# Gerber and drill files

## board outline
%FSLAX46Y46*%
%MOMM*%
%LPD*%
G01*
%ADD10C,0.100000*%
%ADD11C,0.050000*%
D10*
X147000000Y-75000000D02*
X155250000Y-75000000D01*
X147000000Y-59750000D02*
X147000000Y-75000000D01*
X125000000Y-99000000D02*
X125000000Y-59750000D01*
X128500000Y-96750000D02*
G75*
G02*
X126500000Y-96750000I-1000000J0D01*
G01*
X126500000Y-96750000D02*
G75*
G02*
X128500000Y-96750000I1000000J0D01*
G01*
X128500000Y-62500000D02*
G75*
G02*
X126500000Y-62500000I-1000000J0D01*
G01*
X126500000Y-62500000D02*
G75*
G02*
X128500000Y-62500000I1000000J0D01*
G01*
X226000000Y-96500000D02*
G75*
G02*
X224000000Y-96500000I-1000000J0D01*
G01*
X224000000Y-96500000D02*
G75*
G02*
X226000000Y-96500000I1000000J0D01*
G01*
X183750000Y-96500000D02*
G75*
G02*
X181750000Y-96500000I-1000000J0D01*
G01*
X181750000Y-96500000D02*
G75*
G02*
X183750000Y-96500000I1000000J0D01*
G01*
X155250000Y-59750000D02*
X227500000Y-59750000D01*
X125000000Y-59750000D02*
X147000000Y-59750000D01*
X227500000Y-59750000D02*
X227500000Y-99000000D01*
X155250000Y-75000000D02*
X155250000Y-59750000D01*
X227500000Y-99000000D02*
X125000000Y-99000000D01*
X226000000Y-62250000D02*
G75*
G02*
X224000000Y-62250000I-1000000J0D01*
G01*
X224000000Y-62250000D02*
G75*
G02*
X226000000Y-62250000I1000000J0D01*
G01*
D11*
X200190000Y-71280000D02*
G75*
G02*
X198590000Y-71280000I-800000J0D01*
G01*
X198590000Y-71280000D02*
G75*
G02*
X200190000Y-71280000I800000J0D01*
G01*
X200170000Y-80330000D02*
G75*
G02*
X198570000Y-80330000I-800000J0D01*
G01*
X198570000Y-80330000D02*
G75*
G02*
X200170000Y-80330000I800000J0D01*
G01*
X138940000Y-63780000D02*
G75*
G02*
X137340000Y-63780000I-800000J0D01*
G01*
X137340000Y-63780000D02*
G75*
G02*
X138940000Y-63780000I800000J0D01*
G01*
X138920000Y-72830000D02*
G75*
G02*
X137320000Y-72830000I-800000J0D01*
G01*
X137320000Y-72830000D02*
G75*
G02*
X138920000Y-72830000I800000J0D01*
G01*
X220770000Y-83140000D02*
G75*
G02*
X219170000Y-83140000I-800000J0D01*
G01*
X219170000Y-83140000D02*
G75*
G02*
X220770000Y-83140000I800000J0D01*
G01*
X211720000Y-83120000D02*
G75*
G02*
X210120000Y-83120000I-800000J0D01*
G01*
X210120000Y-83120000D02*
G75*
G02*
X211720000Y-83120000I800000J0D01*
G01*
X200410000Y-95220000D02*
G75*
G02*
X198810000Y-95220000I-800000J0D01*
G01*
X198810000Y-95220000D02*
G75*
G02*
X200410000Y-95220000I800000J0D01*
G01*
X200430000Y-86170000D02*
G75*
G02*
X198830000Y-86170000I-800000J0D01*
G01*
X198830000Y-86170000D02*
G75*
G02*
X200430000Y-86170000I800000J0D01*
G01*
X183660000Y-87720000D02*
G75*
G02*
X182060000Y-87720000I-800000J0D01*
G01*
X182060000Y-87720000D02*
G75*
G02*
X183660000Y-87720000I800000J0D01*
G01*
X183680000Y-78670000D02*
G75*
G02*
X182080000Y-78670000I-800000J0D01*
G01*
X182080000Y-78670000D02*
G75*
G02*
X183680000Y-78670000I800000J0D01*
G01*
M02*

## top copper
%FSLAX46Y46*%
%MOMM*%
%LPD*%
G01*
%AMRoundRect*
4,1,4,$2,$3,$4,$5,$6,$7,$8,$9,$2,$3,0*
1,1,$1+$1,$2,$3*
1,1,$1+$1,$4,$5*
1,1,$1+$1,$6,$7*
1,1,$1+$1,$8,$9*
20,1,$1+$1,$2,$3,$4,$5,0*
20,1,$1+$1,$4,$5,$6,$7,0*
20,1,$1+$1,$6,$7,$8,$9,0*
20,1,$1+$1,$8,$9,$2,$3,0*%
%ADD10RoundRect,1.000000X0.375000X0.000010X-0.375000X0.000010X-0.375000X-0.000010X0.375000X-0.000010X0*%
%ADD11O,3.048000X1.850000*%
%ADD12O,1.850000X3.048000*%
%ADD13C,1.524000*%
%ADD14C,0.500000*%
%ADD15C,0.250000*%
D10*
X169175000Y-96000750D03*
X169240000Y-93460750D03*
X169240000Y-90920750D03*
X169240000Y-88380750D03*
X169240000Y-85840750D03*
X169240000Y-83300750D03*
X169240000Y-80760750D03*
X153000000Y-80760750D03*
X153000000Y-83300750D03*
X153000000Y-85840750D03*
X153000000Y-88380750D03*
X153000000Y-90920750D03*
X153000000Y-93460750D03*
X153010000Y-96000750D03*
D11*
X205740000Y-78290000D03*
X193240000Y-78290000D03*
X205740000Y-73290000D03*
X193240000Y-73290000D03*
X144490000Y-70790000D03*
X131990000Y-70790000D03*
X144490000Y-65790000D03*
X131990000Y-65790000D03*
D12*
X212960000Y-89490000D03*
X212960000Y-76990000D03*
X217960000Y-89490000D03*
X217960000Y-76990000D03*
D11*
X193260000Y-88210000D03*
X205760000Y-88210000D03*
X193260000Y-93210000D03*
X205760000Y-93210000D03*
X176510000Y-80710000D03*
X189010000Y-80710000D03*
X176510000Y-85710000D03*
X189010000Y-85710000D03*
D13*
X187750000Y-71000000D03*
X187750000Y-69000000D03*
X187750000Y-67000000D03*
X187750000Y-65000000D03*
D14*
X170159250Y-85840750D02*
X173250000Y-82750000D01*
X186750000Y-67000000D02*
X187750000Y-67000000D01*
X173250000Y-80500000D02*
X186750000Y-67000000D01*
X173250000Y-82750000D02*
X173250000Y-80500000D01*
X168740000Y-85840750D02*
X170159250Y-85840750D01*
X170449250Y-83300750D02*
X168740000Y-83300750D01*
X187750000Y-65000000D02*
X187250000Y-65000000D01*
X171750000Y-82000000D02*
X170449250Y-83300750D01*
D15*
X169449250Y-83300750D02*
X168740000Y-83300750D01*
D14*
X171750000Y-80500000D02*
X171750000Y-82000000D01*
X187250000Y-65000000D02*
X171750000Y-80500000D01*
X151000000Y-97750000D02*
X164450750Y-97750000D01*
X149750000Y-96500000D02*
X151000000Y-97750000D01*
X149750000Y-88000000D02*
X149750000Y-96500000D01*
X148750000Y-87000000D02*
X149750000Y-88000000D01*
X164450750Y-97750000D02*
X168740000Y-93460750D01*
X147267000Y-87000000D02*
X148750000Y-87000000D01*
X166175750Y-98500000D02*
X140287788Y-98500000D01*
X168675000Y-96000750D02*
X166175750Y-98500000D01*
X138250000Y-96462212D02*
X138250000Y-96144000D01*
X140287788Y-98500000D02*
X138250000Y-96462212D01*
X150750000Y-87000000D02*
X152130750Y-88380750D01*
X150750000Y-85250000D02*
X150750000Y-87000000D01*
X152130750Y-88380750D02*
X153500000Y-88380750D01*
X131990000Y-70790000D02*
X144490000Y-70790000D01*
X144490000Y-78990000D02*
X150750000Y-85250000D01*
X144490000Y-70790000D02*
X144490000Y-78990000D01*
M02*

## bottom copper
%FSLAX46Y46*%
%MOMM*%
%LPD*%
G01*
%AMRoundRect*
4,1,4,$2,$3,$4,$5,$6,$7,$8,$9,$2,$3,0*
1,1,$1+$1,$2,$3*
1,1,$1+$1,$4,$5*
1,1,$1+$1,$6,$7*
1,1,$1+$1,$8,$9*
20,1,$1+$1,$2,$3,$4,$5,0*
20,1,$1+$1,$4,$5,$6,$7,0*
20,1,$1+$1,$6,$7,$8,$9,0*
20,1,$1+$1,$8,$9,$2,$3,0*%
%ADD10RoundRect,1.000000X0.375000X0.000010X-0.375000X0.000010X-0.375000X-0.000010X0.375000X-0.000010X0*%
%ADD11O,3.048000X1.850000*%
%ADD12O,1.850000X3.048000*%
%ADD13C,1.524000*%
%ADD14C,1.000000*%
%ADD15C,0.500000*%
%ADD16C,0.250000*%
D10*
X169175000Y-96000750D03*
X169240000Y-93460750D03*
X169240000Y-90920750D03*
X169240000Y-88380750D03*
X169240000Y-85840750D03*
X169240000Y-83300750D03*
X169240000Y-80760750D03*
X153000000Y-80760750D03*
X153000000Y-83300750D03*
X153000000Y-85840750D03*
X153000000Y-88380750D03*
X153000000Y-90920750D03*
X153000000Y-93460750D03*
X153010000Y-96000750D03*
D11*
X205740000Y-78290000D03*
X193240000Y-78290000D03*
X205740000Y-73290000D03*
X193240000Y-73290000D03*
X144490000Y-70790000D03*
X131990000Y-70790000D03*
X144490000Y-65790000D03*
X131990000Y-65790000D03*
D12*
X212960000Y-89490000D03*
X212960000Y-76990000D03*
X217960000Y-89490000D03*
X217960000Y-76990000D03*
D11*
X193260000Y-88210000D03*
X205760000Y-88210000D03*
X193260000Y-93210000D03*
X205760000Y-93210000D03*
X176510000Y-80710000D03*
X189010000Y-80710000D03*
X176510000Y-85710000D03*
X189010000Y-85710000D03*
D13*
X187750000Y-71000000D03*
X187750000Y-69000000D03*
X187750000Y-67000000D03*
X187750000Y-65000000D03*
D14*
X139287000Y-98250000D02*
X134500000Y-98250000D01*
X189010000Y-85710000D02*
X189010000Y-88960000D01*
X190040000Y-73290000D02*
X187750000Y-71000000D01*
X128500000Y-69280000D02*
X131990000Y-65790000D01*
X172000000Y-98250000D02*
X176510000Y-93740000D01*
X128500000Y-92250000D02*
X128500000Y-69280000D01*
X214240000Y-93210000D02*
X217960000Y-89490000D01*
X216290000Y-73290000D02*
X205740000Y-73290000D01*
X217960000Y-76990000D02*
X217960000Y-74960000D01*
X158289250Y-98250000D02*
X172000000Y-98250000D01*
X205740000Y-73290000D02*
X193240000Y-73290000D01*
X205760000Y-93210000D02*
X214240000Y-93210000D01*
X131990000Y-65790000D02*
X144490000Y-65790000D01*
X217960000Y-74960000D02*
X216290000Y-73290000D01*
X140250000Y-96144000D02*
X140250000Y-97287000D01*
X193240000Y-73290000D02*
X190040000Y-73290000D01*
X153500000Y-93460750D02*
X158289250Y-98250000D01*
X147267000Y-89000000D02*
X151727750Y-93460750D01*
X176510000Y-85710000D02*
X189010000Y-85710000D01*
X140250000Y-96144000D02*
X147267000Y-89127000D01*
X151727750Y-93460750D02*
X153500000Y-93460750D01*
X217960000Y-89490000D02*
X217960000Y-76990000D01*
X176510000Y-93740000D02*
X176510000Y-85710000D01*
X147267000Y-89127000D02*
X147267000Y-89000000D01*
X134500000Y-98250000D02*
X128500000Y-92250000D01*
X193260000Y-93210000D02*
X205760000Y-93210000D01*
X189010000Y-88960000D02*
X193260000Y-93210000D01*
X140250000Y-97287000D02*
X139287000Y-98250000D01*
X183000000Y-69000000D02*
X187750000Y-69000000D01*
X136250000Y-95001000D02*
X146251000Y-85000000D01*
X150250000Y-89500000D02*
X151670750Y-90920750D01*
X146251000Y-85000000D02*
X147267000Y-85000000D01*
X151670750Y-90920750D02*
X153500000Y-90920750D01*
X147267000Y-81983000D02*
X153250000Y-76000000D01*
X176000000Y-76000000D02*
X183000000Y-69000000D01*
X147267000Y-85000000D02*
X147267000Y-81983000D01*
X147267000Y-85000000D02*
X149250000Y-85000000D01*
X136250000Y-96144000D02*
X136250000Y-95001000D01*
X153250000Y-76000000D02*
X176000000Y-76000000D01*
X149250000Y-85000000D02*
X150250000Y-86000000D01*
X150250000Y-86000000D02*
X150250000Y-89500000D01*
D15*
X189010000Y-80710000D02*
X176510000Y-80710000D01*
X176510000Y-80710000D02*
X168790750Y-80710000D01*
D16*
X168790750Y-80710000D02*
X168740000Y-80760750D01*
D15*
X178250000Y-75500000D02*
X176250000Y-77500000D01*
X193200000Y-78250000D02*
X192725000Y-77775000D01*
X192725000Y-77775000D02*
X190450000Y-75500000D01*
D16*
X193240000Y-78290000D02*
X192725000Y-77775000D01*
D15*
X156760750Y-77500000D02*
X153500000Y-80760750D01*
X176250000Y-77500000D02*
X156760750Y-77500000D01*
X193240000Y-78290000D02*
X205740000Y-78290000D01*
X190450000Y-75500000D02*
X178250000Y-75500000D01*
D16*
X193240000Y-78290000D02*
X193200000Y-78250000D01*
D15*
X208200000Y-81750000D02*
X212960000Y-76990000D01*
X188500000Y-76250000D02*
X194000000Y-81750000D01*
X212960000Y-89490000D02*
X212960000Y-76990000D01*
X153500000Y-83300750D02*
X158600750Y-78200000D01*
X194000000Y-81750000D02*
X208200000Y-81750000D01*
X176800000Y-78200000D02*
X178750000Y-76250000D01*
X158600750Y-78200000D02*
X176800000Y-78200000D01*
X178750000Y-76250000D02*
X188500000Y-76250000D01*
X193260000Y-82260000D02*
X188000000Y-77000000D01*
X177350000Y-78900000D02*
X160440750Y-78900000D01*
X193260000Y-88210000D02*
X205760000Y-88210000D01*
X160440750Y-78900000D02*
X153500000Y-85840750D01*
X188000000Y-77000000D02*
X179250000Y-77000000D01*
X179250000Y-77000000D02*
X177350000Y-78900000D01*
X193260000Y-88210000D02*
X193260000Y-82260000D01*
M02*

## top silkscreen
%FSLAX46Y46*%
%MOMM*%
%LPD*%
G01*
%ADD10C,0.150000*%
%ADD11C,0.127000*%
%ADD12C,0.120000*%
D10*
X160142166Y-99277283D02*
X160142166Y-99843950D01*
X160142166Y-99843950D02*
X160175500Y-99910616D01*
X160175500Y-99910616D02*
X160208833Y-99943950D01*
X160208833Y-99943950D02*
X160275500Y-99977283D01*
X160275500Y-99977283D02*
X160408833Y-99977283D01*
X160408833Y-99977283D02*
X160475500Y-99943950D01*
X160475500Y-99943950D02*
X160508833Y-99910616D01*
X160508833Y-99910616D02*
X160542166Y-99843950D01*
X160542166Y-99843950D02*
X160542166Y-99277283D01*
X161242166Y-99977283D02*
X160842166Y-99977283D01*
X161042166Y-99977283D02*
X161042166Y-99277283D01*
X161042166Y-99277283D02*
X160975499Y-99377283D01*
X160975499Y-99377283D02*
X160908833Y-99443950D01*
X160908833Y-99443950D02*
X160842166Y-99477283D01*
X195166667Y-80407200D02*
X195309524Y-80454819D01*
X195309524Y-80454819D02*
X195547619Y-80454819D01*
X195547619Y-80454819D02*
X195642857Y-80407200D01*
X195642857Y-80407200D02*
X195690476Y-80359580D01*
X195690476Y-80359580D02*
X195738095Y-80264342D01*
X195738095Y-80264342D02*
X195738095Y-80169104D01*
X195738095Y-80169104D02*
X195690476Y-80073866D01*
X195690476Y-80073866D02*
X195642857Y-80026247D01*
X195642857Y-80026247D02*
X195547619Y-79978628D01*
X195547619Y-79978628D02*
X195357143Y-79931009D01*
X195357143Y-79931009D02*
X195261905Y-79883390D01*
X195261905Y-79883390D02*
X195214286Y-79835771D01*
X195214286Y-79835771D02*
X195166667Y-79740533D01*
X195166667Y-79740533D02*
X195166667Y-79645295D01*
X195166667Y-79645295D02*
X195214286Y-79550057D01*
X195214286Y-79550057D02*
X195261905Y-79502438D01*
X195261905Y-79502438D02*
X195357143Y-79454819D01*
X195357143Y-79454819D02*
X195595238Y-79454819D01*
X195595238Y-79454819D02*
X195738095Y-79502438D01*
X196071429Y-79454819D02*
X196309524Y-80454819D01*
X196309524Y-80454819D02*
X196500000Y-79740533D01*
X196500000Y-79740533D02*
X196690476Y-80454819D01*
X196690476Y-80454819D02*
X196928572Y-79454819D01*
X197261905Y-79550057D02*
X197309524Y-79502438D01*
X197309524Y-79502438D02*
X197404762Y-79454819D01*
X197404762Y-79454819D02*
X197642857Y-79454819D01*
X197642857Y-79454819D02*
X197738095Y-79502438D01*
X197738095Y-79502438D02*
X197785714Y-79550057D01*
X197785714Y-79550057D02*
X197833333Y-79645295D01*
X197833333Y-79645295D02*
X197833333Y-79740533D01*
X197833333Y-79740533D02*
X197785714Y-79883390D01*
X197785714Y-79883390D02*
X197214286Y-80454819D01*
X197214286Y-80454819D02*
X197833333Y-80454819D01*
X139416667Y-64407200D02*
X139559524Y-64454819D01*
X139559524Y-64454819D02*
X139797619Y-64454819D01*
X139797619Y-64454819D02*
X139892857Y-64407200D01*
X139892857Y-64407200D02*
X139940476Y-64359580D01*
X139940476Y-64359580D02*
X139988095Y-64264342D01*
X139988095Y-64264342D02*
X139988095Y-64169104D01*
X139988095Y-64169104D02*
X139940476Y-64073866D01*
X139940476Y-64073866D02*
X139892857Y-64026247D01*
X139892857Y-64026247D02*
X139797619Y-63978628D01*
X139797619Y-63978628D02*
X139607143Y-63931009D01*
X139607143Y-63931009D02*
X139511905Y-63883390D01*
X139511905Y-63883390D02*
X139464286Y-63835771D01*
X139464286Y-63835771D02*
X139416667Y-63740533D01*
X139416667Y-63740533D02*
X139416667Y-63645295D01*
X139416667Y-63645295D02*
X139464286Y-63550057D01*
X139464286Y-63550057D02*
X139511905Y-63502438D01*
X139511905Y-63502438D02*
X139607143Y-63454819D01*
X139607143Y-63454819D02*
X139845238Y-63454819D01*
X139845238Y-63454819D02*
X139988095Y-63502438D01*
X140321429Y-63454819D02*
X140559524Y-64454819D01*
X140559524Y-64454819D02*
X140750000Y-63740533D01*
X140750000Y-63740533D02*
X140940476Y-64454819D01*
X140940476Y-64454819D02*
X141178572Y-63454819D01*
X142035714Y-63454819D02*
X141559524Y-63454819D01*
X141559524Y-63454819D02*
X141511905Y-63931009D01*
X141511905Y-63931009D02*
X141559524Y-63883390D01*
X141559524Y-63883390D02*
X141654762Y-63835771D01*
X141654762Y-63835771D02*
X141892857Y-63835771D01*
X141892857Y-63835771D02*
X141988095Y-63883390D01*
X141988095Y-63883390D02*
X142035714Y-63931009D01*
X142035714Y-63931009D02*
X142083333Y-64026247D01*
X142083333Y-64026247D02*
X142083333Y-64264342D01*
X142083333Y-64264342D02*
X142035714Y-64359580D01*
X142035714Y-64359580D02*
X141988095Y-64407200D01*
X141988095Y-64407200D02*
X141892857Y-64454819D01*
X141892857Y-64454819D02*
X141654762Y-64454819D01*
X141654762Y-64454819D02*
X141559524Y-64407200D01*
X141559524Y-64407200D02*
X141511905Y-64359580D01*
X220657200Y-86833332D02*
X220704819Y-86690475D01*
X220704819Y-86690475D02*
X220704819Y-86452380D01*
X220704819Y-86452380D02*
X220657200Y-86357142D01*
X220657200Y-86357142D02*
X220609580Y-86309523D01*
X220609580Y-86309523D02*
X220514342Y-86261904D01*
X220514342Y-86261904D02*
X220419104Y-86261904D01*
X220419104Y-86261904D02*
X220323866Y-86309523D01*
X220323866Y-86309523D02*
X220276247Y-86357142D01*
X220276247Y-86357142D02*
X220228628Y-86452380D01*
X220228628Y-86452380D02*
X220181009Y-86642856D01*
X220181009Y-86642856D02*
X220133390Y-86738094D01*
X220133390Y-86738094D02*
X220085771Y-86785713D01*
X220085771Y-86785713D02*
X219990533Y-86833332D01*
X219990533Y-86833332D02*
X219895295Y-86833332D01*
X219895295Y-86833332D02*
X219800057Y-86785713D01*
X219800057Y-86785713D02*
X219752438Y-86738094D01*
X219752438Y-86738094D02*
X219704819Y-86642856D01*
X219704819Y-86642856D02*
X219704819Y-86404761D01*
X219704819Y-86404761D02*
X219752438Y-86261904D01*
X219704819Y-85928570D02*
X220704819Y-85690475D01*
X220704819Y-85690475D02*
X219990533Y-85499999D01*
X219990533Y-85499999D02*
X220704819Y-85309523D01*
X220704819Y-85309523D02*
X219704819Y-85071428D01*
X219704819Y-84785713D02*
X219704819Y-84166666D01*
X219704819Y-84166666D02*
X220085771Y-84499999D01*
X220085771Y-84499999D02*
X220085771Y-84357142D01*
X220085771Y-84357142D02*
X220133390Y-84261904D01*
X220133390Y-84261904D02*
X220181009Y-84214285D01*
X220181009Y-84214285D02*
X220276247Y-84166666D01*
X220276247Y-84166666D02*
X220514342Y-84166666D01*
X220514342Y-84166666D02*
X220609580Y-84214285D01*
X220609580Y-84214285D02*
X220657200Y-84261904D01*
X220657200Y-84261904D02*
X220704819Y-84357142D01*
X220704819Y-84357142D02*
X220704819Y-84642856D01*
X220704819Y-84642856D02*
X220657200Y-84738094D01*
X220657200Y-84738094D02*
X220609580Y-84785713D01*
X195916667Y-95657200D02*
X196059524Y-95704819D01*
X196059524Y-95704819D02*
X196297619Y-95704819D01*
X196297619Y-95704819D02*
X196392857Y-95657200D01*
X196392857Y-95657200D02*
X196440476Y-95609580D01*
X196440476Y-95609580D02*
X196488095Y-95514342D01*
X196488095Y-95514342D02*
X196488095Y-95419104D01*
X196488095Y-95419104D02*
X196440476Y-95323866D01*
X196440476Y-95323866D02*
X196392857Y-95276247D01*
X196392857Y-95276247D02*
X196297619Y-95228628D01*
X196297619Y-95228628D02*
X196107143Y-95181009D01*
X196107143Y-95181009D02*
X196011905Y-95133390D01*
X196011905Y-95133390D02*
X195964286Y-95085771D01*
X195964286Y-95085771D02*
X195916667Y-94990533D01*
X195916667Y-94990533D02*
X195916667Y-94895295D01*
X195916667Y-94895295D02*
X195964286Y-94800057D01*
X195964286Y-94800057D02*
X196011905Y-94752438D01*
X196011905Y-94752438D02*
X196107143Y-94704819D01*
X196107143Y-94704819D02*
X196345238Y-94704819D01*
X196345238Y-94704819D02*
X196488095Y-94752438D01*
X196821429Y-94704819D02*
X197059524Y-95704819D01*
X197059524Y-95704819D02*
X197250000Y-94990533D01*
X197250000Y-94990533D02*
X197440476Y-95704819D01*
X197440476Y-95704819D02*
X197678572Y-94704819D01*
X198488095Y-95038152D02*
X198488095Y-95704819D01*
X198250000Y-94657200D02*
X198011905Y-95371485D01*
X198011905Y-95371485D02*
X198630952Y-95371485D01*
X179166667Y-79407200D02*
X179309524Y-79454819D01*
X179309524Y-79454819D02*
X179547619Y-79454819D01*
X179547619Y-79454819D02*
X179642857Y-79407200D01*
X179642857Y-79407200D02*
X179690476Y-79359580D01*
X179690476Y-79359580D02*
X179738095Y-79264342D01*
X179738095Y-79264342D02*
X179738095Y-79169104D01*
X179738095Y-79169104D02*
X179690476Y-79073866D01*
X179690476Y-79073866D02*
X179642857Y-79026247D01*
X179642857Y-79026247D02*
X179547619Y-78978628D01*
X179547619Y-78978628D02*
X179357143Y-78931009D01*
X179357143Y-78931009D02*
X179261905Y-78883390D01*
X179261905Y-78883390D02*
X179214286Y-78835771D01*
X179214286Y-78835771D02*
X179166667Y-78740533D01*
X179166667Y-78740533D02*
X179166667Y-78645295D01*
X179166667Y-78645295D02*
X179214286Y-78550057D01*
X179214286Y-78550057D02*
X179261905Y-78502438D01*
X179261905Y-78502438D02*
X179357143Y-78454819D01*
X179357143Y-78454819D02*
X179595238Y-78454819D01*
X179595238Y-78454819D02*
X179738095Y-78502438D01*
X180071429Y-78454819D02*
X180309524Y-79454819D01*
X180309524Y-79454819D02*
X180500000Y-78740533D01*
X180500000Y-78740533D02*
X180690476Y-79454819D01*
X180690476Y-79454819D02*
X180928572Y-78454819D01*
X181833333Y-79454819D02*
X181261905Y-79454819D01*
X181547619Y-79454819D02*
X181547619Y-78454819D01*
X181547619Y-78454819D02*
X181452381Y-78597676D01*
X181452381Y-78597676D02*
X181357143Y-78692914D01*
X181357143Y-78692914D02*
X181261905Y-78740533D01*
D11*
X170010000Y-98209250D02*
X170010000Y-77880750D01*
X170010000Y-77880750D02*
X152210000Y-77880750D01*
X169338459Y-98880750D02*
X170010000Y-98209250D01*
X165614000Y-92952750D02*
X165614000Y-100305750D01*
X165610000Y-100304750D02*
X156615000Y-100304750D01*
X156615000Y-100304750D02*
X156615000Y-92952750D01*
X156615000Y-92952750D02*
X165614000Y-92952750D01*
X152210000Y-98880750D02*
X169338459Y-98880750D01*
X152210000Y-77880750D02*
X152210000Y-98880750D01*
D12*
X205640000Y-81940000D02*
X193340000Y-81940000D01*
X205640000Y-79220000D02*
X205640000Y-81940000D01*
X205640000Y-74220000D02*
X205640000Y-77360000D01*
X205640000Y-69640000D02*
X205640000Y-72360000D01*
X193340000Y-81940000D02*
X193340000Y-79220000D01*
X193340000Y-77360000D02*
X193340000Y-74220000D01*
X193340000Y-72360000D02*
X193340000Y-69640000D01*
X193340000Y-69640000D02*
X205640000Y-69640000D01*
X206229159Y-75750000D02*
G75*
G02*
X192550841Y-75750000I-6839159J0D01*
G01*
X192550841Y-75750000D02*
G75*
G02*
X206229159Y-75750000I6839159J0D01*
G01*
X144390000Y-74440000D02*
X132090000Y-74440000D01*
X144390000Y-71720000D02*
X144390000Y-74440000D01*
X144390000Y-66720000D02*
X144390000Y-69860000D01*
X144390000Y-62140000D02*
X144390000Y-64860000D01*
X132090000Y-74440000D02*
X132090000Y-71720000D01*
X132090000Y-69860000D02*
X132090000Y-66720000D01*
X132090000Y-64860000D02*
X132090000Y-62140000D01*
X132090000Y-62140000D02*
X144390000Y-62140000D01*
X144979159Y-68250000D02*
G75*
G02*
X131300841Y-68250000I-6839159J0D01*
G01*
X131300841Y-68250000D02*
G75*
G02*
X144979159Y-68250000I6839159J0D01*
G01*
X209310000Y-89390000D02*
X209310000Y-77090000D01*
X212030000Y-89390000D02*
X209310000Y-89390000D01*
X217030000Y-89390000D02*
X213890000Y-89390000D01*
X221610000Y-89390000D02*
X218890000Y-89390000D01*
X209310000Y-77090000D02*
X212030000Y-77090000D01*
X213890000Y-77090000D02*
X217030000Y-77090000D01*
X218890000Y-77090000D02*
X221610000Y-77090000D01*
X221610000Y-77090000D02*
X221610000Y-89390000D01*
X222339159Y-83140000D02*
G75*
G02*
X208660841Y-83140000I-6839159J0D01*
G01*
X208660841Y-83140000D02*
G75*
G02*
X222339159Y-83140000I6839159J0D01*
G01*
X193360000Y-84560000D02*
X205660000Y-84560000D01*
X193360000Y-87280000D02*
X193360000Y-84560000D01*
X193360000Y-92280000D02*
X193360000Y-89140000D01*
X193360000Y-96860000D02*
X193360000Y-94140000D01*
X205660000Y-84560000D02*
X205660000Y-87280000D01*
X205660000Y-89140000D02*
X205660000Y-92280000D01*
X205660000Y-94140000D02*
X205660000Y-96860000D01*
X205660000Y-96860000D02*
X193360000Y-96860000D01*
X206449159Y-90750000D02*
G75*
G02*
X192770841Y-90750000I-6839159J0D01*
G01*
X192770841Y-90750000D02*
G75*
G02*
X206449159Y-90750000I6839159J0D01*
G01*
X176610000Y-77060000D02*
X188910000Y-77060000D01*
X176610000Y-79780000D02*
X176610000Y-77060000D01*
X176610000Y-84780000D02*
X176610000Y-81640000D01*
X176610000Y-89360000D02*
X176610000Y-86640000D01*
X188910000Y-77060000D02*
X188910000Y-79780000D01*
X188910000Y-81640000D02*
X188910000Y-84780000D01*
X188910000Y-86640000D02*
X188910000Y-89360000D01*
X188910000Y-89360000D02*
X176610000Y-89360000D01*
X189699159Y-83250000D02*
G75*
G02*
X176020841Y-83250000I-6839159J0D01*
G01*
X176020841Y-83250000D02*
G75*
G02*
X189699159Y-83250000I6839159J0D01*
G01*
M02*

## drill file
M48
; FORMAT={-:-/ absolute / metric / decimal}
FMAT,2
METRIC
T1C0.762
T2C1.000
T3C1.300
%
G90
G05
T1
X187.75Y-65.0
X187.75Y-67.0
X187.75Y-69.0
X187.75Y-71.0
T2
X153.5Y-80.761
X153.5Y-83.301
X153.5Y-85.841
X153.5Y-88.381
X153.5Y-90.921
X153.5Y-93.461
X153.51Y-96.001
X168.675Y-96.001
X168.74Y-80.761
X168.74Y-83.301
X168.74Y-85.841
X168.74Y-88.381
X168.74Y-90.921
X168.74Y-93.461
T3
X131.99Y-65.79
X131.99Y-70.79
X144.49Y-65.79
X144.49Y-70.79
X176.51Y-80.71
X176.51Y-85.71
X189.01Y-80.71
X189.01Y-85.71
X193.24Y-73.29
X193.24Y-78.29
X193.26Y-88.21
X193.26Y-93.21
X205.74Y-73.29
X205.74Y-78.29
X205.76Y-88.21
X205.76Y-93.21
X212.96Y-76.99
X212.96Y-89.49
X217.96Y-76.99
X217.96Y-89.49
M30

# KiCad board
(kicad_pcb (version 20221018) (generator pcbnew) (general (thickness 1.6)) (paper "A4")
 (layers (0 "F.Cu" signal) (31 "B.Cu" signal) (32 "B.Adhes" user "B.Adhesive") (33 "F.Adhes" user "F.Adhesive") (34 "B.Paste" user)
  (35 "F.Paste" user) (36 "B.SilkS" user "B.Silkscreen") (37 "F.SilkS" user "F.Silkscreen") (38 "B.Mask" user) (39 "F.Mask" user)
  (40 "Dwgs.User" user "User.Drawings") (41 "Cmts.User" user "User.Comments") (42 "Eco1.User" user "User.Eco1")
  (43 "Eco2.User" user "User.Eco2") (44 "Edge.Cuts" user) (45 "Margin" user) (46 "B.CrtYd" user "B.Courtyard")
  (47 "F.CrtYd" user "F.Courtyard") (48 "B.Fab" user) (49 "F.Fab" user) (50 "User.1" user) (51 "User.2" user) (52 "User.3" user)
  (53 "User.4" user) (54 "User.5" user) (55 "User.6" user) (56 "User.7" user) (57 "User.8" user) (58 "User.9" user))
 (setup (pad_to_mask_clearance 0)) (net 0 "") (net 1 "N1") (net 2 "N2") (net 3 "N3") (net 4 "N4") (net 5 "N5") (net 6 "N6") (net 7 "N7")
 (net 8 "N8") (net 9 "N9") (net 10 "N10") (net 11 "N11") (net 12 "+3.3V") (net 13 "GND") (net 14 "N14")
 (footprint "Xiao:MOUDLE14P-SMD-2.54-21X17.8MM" (layer "F.Cu") (at 170.01 77.88075 180)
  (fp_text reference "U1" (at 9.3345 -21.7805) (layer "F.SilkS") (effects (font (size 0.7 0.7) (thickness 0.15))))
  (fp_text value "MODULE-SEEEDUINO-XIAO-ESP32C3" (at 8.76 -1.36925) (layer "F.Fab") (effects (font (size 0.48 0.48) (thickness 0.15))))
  (fp_line (start 0 -20.3285) (end 0 0) (stroke (width 0.127) (type solid)) (layer "F.SilkS"))
  (fp_line (start 0 0) (end 17.8 0) (stroke (width 0.127) (type solid)) (layer "F.SilkS"))
  (fp_line (start 0.671541 -21) (end 0 -20.3285) (stroke (width 0.127) (type solid)) (layer "F.SilkS"))
  (fp_line (start 4.396 -15.072) (end 4.396 -22.425) (stroke (width 0.127) (type solid)) (layer "F.SilkS"))
  (fp_line (start 4.4 -22.424) (end 13.395 -22.424) (stroke (width 0.127) (type solid)) (layer "F.SilkS"))
  (fp_line (start 13.395 -22.424) (end 13.395 -15.072) (stroke (width 0.127) (type solid)) (layer "F.SilkS"))
  (fp_line (start 13.395 -15.072) (end 4.396 -15.072) (stroke (width 0.127) (type solid)) (layer "F.SilkS"))
  (fp_line (start 17.8 -21) (end 0.671541 -21) (stroke (width 0.127) (type solid)) (layer "F.SilkS"))
  (fp_line (start 17.8 0) (end 17.8 -21) (stroke (width 0.127) (type solid)) (layer "F.SilkS"))
  (pad "1" thru_hole roundrect (at 1.335 -18.12 180) (size 2.75 2) (drill 1 (offset -0.5 0)) (layers "*.Cu" "*.Mask") (roundrect_rratio 0.5)
   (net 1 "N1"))
  (pad "2" thru_hole roundrect (at 1.27 -15.58 180) (size 2.75 2) (drill 1 (offset -0.5 0)) (layers "*.Cu" "*.Mask") (roundrect_rratio 0.5)
   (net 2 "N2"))
  (pad "3" thru_hole roundrect (at 1.27 -13.04 180) (size 2.75 2) (drill 1 (offset -0.5 0)) (layers "*.Cu" "*.Mask") (roundrect_rratio 0.5)
   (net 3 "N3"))
  (pad "4" thru_hole roundrect (at 1.27 -10.5 180) (size 2.75 2) (drill 1 (offset -0.5 0)) (layers "*.Cu" "*.Mask") (roundrect_rratio 0.5)
   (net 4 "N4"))
  (pad "5" thru_hole roundrect (at 1.27 -7.96 180) (size 2.75 2) (drill 1 (offset -0.5 0)) (layers "*.Cu" "*.Mask") (roundrect_rratio 0.5)
   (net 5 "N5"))
  (pad "6" thru_hole roundrect (at 1.27 -5.42 180) (size 2.75 2) (drill 1 (offset -0.5 0)) (layers "*.Cu" "*.Mask") (roundrect_rratio 0.5)
   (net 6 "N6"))
  (pad "7" thru_hole roundrect (at 1.27 -2.88 180) (size 2.75 2) (drill 1 (offset -0.5 0)) (layers "*.Cu" "*.Mask") (roundrect_rratio 0.5)
   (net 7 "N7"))
  (pad "8" thru_hole roundrect (at 16.51 -2.88 180) (size 2.75 2) (drill 1 (offset 0.5 0)) (layers "*.Cu" "*.Mask") (roundrect_rratio 0.5)
   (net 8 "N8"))
  (pad "9" thru_hole roundrect (at 16.51 -5.42 180) (size 2.75 2) (drill 1 (offset 0.5 0)) (layers "*.Cu" "*.Mask") (roundrect_rratio 0.5)
   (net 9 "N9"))
  (pad "10" thru_hole roundrect (at 16.51 -7.96 180) (size 2.75 2) (drill 1 (offset 0.5 0)) (layers "*.Cu" "*.Mask") (roundrect_rratio 0.5)
   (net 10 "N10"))
  (pad "11" thru_hole roundrect (at 16.51 -10.5 180) (size 2.75 2) (drill 1 (offset 0.5 0)) (layers "*.Cu" "*.Mask") (roundrect_rratio 0.5)
   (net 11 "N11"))
  (pad "12" thru_hole roundrect (at 16.51 -13.04 180) (size 2.75 2) (drill 1 (offset 0.5 0)) (layers "*.Cu" "*.Mask") (roundrect_rratio 0.5)
   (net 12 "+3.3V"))
  (pad "13" thru_hole roundrect (at 16.51 -15.58 180) (size 2.75 2) (drill 1 (offset 0.5 0)) (layers "*.Cu" "*.Mask") (roundrect_rratio 0.5)
   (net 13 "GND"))
  (pad "14" thru_hole roundrect (at 16.5 -18.12 180) (size 2.75 2) (drill 1 (offset 0.5 0)) (layers "*.Cu" "*.Mask") (roundrect_rratio 0.5)
   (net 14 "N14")))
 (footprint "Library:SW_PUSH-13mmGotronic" (layer "F.Cu") (at 205.74 78.29 180)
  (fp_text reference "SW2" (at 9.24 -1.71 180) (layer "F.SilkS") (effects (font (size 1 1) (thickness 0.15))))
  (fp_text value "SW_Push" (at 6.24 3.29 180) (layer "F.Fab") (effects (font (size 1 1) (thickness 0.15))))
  (fp_line (start 0.1 -3.65) (end 12.4 -3.65) (stroke (width 0.12) (type solid)) (layer "F.SilkS"))
  (fp_line (start 0.1 -0.93) (end 0.1 -3.65) (stroke (width 0.12) (type solid)) (layer "F.SilkS"))
  (fp_line (start 0.1 4.07) (end 0.1 0.93) (stroke (width 0.12) (type solid)) (layer "F.SilkS"))
  (fp_line (start 0.1 8.65) (end 0.1 5.93) (stroke (width 0.12) (type solid)) (layer "F.SilkS"))
  (fp_line (start 12.4 -3.65) (end 12.4 -0.93) (stroke (width 0.12) (type solid)) (layer "F.SilkS"))
  (fp_line (start 12.4 0.93) (end 12.4 4.07) (stroke (width 0.12) (type solid)) (layer "F.SilkS"))
  (fp_line (start 12.4 5.93) (end 12.4 8.65) (stroke (width 0.12) (type solid)) (layer "F.SilkS"))
  (fp_line (start 12.4 8.65) (end 0.1 8.65) (stroke (width 0.12) (type solid)) (layer "F.SilkS"))
  (fp_circle (center 6.35 2.54) (end 12.7 5.08) (stroke (width 0.12) (type solid)) (fill none) (layer "F.SilkS"))
  (fp_circle (center 6.35 7.01) (end 7.15 7.01) (stroke (width 0.05) (type default)) (fill none) (layer "Edge.Cuts"))
  (fp_circle (center 6.37 -2.04) (end 7.17 -2.04) (stroke (width 0.05) (type default)) (fill none) (layer "Edge.Cuts"))
  (pad "1" thru_hole oval (at 0 0 180) (size 3.048 1.85) (drill 1.3) (layers "*.Cu" "*.Mask") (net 8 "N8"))
  (pad "1" thru_hole oval (at 12.5 0 180) (size 3.048 1.85) (drill 1.3) (layers "*.Cu" "*.Mask") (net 8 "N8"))
  (pad "2" thru_hole oval (at 0 5 180) (size 3.048 1.85) (drill 1.3) (layers "*.Cu" "*.Mask") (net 13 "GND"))
  (pad "2" thru_hole oval (at 12.5 5 180) (size 3.048 1.85) (drill 1.3) (layers "*.Cu" "*.Mask") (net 13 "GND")))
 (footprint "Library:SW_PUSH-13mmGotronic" (layer "F.Cu") (at 144.49 70.79 180)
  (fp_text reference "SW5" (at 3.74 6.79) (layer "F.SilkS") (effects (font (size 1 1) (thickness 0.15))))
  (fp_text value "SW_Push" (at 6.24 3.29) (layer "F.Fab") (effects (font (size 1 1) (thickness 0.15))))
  (fp_line (start 0.1 -3.65) (end 12.4 -3.65) (stroke (width 0.12) (type solid)) (layer "F.SilkS"))
  (fp_line (start 0.1 -0.93) (end 0.1 -3.65) (stroke (width 0.12) (type solid)) (layer "F.SilkS"))
  (fp_line (start 0.1 4.07) (end 0.1 0.93) (stroke (width 0.12) (type solid)) (layer "F.SilkS"))
  (fp_line (start 0.1 8.65) (end 0.1 5.93) (stroke (width 0.12) (type solid)) (layer "F.SilkS"))
  (fp_line (start 12.4 -3.65) (end 12.4 -0.93) (stroke (width 0.12) (type solid)) (layer "F.SilkS"))
  (fp_line (start 12.4 0.93) (end 12.4 4.07) (stroke (width 0.12) (type solid)) (layer "F.SilkS"))
  (fp_line (start 12.4 5.93) (end 12.4 8.65) (stroke (width 0.12) (type solid)) (layer "F.SilkS"))
  (fp_line (start 12.4 8.65) (end 0.1 8.65) (stroke (width 0.12) (type solid)) (layer "F.SilkS"))
  (fp_circle (center 6.35 2.54) (end 12.7 5.08) (stroke (width 0.12) (type solid)) (fill none) (layer "F.SilkS"))
  (fp_circle (center 6.35 7.01) (end 7.15 7.01) (stroke (width 0.05) (type default)) (fill none) (layer "Edge.Cuts"))
  (fp_circle (center 6.37 -2.04) (end 7.17 -2.04) (stroke (width 0.05) (type default)) (fill none) (layer "Edge.Cuts"))
  (pad "1" thru_hole oval (at 0 0 180) (size 3.048 1.85) (drill 1.3) (layers "*.Cu" "*.Mask") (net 11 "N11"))
  (pad "1" thru_hole oval (at 12.5 0 180) (size 3.048 1.85) (drill 1.3) (layers "*.Cu" "*.Mask") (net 11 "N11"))
  (pad "2" thru_hole oval (at 0 5 180) (size 3.048 1.85) (drill 1.3) (layers "*.Cu" "*.Mask") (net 13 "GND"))
  (pad "2" thru_hole oval (at 12.5 5 180) (size 3.048 1.85) (drill 1.3) (layers "*.Cu" "*.Mask") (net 13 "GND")))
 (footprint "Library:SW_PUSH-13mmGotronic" (layer "F.Cu") (at 212.96 89.49 90)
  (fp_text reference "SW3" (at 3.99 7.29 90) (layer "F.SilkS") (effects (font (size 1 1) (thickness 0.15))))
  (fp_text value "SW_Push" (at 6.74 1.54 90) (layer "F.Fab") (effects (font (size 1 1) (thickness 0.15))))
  (fp_line (start 0.1 -3.65) (end 12.4 -3.65) (stroke (width 0.12) (type solid)) (layer "F.SilkS"))
  (fp_line (start 0.1 -0.93) (end 0.1 -3.65) (stroke (width 0.12) (type solid)) (layer "F.SilkS"))
  (fp_line (start 0.1 4.07) (end 0.1 0.93) (stroke (width 0.12) (type solid)) (layer "F.SilkS"))
  (fp_line (start 0.1 8.65) (end 0.1 5.93) (stroke (width 0.12) (type solid)) (layer "F.SilkS"))
  (fp_line (start 12.4 -3.65) (end 12.4 -0.93) (stroke (width 0.12) (type solid)) (layer "F.SilkS"))
  (fp_line (start 12.4 0.93) (end 12.4 4.07) (stroke (width 0.12) (type solid)) (layer "F.SilkS"))
  (fp_line (start 12.4 5.93) (end 12.4 8.65) (stroke (width 0.12) (type solid)) (layer "F.SilkS"))
  (fp_line (start 12.4 8.65) (end 0.1 8.65) (stroke (width 0.12) (type solid)) (layer "F.SilkS"))
  (fp_circle (center 6.35 2.54) (end 12.7 5.08) (stroke (width 0.12) (type solid)) (fill none) (layer "F.SilkS"))
  (fp_circle (center 6.35 7.01) (end 7.15 7.01) (stroke (width 0.05) (type default)) (fill none) (layer "Edge.Cuts"))
  (fp_circle (center 6.37 -2.04) (end 7.17 -2.04) (stroke (width 0.05) (type default)) (fill none) (layer "Edge.Cuts"))
  (pad "1" thru_hole oval (at 0 0 90) (size 3.048 1.85) (drill 1.3) (layers "*.Cu" "*.Mask") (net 9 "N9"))
  (pad "1" thru_hole oval (at 12.5 0 90) (size 3.048 1.85) (drill 1.3) (layers "*.Cu" "*.Mask") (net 9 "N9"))
  (pad "2" thru_hole oval (at 0 5 90) (size 3.048 1.85) (drill 1.3) (layers "*.Cu" "*.Mask") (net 13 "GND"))
  (pad "2" thru_hole oval (at 12.5 5 90) (size 3.048 1.85) (drill 1.3) (layers "*.Cu" "*.Mask") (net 13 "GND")))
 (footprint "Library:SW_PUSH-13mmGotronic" (layer "F.Cu") (at 193.26 88.21)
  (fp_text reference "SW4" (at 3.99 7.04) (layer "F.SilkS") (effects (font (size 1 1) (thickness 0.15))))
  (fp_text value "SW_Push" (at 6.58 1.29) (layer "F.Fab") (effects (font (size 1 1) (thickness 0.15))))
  (fp_line (start 0.1 -3.65) (end 12.4 -3.65) (stroke (width 0.12) (type solid)) (layer "F.SilkS"))
  (fp_line (start 0.1 -0.93) (end 0.1 -3.65) (stroke (width 0.12) (type solid)) (layer "F.SilkS"))
  (fp_line (start 0.1 4.07) (end 0.1 0.93) (stroke (width 0.12) (type solid)) (layer "F.SilkS"))
  (fp_line (start 0.1 8.65) (end 0.1 5.93) (stroke (width 0.12) (type solid)) (layer "F.SilkS"))
  (fp_line (start 12.4 -3.65) (end 12.4 -0.93) (stroke (width 0.12) (type solid)) (layer "F.SilkS"))
  (fp_line (start 12.4 0.93) (end 12.4 4.07) (stroke (width 0.12) (type solid)) (layer "F.SilkS"))
  (fp_line (start 12.4 5.93) (end 12.4 8.65) (stroke (width 0.12) (type solid)) (layer "F.SilkS"))
  (fp_line (start 12.4 8.65) (end 0.1 8.65) (stroke (width 0.12) (type solid)) (layer "F.SilkS"))
  (fp_circle (center 6.35 2.54) (end 12.7 5.08) (stroke (width 0.12) (type solid)) (fill none) (layer "F.SilkS"))
  (fp_circle (center 6.35 7.01) (end 7.15 7.01) (stroke (width 0.05) (type default)) (fill none) (layer "Edge.Cuts"))
  (fp_circle (center 6.37 -2.04) (end 7.17 -2.04) (stroke (width 0.05) (type default)) (fill none) (layer "Edge.Cuts"))
  (pad "1" thru_hole oval (at 0 0) (size 3.048 1.85) (drill 1.3) (layers "*.Cu" "*.Mask") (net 10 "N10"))
  (pad "1" thru_hole oval (at 12.5 0) (size 3.048 1.85) (drill 1.3) (layers "*.Cu" "*.Mask") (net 10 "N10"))
  (pad "2" thru_hole oval (at 0 5) (size 3.048 1.85) (drill 1.3) (layers "*.Cu" "*.Mask") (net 13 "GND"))
  (pad "2" thru_hole oval (at 12.5 5) (size 3.048 1.85) (drill 1.3) (layers "*.Cu" "*.Mask") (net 13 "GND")))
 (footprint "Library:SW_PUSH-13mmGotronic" (layer "F.Cu") (at 176.51 80.71)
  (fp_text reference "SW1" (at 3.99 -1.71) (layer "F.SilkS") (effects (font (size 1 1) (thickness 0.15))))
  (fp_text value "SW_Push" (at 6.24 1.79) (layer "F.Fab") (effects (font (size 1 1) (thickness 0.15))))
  (fp_line (start 0.1 -3.65) (end 12.4 -3.65) (stroke (width 0.12) (type solid)) (layer "F.SilkS"))
  (fp_line (start 0.1 -0.93) (end 0.1 -3.65) (stroke (width 0.12) (type solid)) (layer "F.SilkS"))
  (fp_line (start 0.1 4.07) (end 0.1 0.93) (stroke (width 0.12) (type solid)) (layer "F.SilkS"))
  (fp_line (start 0.1 8.65) (end 0.1 5.93) (stroke (width 0.12) (type solid)) (layer "F.SilkS"))
  (fp_line (start 12.4 -3.65) (end 12.4 -0.93) (stroke (width 0.12) (type solid)) (layer "F.SilkS"))
  (fp_line (start 12.4 0.93) (end 12.4 4.07) (stroke (width 0.12) (type solid)) (layer "F.SilkS"))
  (fp_line (start 12.4 5.93) (end 12.4 8.65) (stroke (width 0.12) (type solid)) (layer "F.SilkS"))
  (fp_line (start 12.4 8.65) (end 0.1 8.65) (stroke (width 0.12) (type solid)) (layer "F.SilkS"))
  (fp_circle (center 6.35 2.54) (end 12.7 5.08) (stroke (width 0.12) (type solid)) (fill none) (layer "F.SilkS"))
  (fp_circle (center 6.35 7.01) (end 7.15 7.01) (stroke (width 0.05) (type default)) (fill none) (layer "Edge.Cuts"))
  (fp_circle (center 6.37 -2.04) (end 7.17 -2.04) (stroke (width 0.05) (type default)) (fill none) (layer "Edge.Cuts"))
  (pad "1" thru_hole oval (at 0 0) (size 3.048 1.85) (drill 1.3) (layers "*.Cu" "*.Mask") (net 7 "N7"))
  (pad "1" thru_hole oval (at 12.5 0) (size 3.048 1.85) (drill 1.3) (layers "*.Cu" "*.Mask") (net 7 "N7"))
  (pad "2" thru_hole oval (at 0 5) (size 3.048 1.85) (drill 1.3) (layers "*.Cu" "*.Mask") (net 13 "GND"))
  (pad "2" thru_hole oval (at 12.5 5) (size 3.048 1.85) (drill 1.3) (layers "*.Cu" "*.Mask") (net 13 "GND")))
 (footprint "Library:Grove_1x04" (layer "B.Cu") (at 187.75 71)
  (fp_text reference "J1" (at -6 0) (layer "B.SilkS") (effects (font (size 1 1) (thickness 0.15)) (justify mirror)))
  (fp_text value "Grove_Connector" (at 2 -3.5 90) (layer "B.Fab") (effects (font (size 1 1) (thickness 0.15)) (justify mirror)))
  (pad "1" thru_hole circle (at 0 0) (size 1.524 1.524) (drill 0.762) (layers "*.Cu" "*.Mask" "B.SilkS") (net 13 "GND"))
  (pad "2" thru_hole circle (at 0 -2) (size 1.524 1.524) (drill 0.762) (layers "*.Cu" "*.Mask" "B.SilkS") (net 12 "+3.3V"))
  (pad "3" thru_hole circle (at 0 -4) (size 1.524 1.524) (drill 0.762) (layers "*.Cu" "*.Mask" "B.SilkS") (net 5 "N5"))
  (pad "4" thru_hole circle (at 0 -6) (size 1.524 1.524) (drill 0.762) (layers "*.Cu" "*.Mask" "B.SilkS") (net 6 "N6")))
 (gr_line (start 147 75) (end 155.25 75) (stroke (width 0.1) (type default)) (layer "Edge.Cuts"))
 (gr_line (start 147 59.75) (end 147 75) (stroke (width 0.1) (type default)) (layer "Edge.Cuts"))
 (gr_line (start 125 99) (end 125 59.75) (stroke (width 0.1) (type default)) (layer "Edge.Cuts"))
 (gr_circle (center 127.5 96.75) (end 128.5 96.75) (stroke (width 0.1) (type default)) (fill none) (layer "Edge.Cuts"))
 (gr_circle (center 127.5 62.5) (end 128.5 62.5) (stroke (width 0.1) (type default)) (fill none) (layer "Edge.Cuts"))
 (gr_circle (center 225 96.5) (end 226 96.5) (stroke (width 0.1) (type default)) (fill none) (layer "Edge.Cuts"))
 (gr_circle (center 182.75 96.5) (end 183.75 96.5) (stroke (width 0.1) (type default)) (fill none) (layer "Edge.Cuts"))
 (gr_line (start 155.25 59.75) (end 227.5 59.75) (stroke (width 0.1) (type default)) (layer "Edge.Cuts"))
 (gr_line (start 125 59.75) (end 147 59.75) (stroke (width 0.1) (type default)) (layer "Edge.Cuts"))
 (gr_rect (start 177 104.75) (end 177 104.75) (stroke (width 0.1) (type default)) (fill none) (layer "Edge.Cuts"))
 (gr_line (start 227.5 59.75) (end 227.5 99) (stroke (width 0.1) (type default)) (layer "Edge.Cuts"))
 (gr_line (start 155.25 75) (end 155.25 59.75) (stroke (width 0.1) (type default)) (layer "Edge.Cuts"))
 (gr_line (start 227.5 99) (end 125 99) (stroke (width 0.1) (type default)) (layer "Edge.Cuts"))
 (gr_circle (center 225 62.25) (end 226 62.25) (stroke (width 0.1) (type default)) (fill none) (layer "Edge.Cuts"))
 (segment (start 139.287 98.25) (end 134.5 98.25) (width 1) (layer "B.Cu") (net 13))
 (segment (start 189.01 85.71) (end 189.01 88.96) (width 1) (layer "B.Cu") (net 13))
 (segment (start 190.04 73.29) (end 187.75 71) (width 1) (layer "B.Cu") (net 13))
 (segment (start 128.5 69.28) (end 131.99 65.79) (width 1) (layer "B.Cu") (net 13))
 (segment (start 172 98.25) (end 176.51 93.74) (width 1) (layer "B.Cu") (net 13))
 (segment (start 128.5 92.25) (end 128.5 69.28) (width 1) (layer "B.Cu") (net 13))
 (segment (start 214.24 93.21) (end 217.96 89.49) (width 1) (layer "B.Cu") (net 13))
 (segment (start 216.29 73.29) (end 205.74 73.29) (width 1) (layer "B.Cu") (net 13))
 (segment (start 217.96 76.99) (end 217.96 74.96) (width 1) (layer "B.Cu") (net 13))
 (segment (start 158.28925 98.25) (end 172 98.25) (width 1) (layer "B.Cu") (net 13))
 (segment (start 205.74 73.29) (end 193.24 73.29) (width 1) (layer "B.Cu") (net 13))
 (segment (start 205.76 93.21) (end 214.24 93.21) (width 1) (layer "B.Cu") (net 13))
 (segment (start 131.99 65.79) (end 144.49 65.79) (width 1) (layer "B.Cu") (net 13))
 (segment (start 217.96 74.96) (end 216.29 73.29) (width 1) (layer "B.Cu") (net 13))
 (segment (start 140.25 96.144) (end 140.25 97.287) (width 1) (layer "B.Cu") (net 13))
 (segment (start 193.24 73.29) (end 190.04 73.29) (width 1) (layer "B.Cu") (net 13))
 (segment (start 153.5 93.46075) (end 158.28925 98.25) (width 1) (layer "B.Cu") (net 13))
 (segment (start 147.267 89) (end 151.72775 93.46075) (width 1) (layer "B.Cu") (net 13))
 (segment (start 176.51 85.71) (end 189.01 85.71) (width 1) (layer "B.Cu") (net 13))
 (segment (start 140.25 96.144) (end 147.267 89.127) (width 1) (layer "B.Cu") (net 13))
 (segment (start 151.72775 93.46075) (end 153.5 93.46075) (width 1) (layer "B.Cu") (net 13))
 (segment (start 217.96 89.49) (end 217.96 76.99) (width 1) (layer "B.Cu") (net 13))
 (segment (start 176.51 93.74) (end 176.51 85.71) (width 1) (layer "B.Cu") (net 13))
 (segment (start 147.267 89.127) (end 147.267 89) (width 1) (layer "B.Cu") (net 13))
 (segment (start 134.5 98.25) (end 128.5 92.25) (width 1) (layer "B.Cu") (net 13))
 (segment (start 193.26 93.21) (end 205.76 93.21) (width 1) (layer "B.Cu") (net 13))
 (segment (start 189.01 88.96) (end 193.26 93.21) (width 1) (layer "B.Cu") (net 13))
 (segment (start 140.25 97.287) (end 139.287 98.25) (width 1) (layer "B.Cu") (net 13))
 (segment (start 183 69) (end 187.75 69) (width 1) (layer "B.Cu") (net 12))
 (segment (start 136.25 95.001) (end 146.251 85) (width 1) (layer "B.Cu") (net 12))
 (segment (start 150.25 89.5) (end 151.67075 90.92075) (width 1) (layer "B.Cu") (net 12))
 (segment (start 146.251 85) (end 147.267 85) (width 1) (layer "B.Cu") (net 12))
 (segment (start 151.67075 90.92075) (end 153.5 90.92075) (width 1) (layer "B.Cu") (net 12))
 (segment (start 147.267 81.983) (end 153.25 76) (width 1) (layer "B.Cu") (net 12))
 (segment (start 176 76) (end 183 69) (width 1) (layer "B.Cu") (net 12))
 (segment (start 147.267 85) (end 147.267 81.983) (width 1) (layer "B.Cu") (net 12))
 (segment (start 147.267 85) (end 149.25 85) (width 1) (layer "B.Cu") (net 12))
 (segment (start 136.25 96.144) (end 136.25 95.001) (width 1) (layer "B.Cu") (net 12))
 (segment (start 153.25 76) (end 176 76) (width 1) (layer "B.Cu") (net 12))
 (segment (start 149.25 85) (end 150.25 86) (width 1) (layer "B.Cu") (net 12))
 (segment (start 150.25 86) (end 150.25 89.5) (width 1) (layer "B.Cu") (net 12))
 (segment (start 170.15925 85.84075) (end 173.25 82.75) (width 0.5) (layer "F.Cu") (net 5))
 (segment (start 186.75 67) (end 187.75 67) (width 0.5) (layer "F.Cu") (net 5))
 (segment (start 173.25 80.5) (end 186.75 67) (width 0.5) (layer "F.Cu") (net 5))
 (segment (start 173.25 82.75) (end 173.25 80.5) (width 0.5) (layer "F.Cu") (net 5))
 (segment (start 168.74 85.84075) (end 170.15925 85.84075) (width 0.5) (layer "F.Cu") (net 5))
 (segment (start 170.44925 83.30075) (end 168.74 83.30075) (width 0.5) (layer "F.Cu") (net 6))
 (segment (start 187.75 65) (end 187.25 65) (width 0.5) (layer "F.Cu") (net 6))
 (segment (start 171.75 82) (end 170.44925 83.30075) (width 0.5) (layer "F.Cu") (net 6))
 (segment (start 169.44925 83.30075) (end 168.74 83.30075) (width 0.25) (layer "F.Cu") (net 6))
 (segment (start 171.75 80.5) (end 171.75 82) (width 0.5) (layer "F.Cu") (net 6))
 (segment (start 187.25 65) (end 171.75 80.5) (width 0.5) (layer "F.Cu") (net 6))
 (segment (start 151 97.75) (end 164.45075 97.75) (width 0.5) (layer "F.Cu") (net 2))
 (segment (start 149.75 96.5) (end 151 97.75) (width 0.5) (layer "F.Cu") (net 2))
 (segment (start 149.75 88) (end 149.75 96.5) (width 0.5) (layer "F.Cu") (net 2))
 (segment (start 148.75 87) (end 149.75 88) (width 0.5) (layer "F.Cu") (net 2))
 (segment (start 164.45075 97.75) (end 168.74 93.46075) (width 0.5) (layer "F.Cu") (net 2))
 (segment (start 147.267 87) (end 148.75 87) (width 0.5) (layer "F.Cu") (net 2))
 (segment (start 166.17575 98.5) (end 140.287788 98.5) (width 0.5) (layer "F.Cu") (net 1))
 (segment (start 168.675 96.00075) (end 166.17575 98.5) (width 0.5) (layer "F.Cu") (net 1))
 (segment (start 138.25 96.462212) (end 138.25 96.144) (width 0.5) (layer "F.Cu") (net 1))
 (segment (start 140.287788 98.5) (end 138.25 96.462212) (width 0.5) (layer "F.Cu") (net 1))
 (segment (start 189.01 80.71) (end 176.51 80.71) (width 0.5) (layer "B.Cu") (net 7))
 (segment (start 176.51 80.71) (end 168.79075 80.71) (width 0.5) (layer "B.Cu") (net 7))
 (segment (start 168.79075 80.71) (end 168.74 80.76075) (width 0.25) (layer "B.Cu") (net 7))
 (segment (start 178.25 75.5) (end 176.25 77.5) (width 0.5) (layer "B.Cu") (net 8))
 (segment (start 193.2 78.25) (end 192.725 77.775) (width 0.5) (layer "B.Cu") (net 8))
 (segment (start 192.725 77.775) (end 190.45 75.5) (width 0.5) (layer "B.Cu") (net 8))
 (segment (start 193.24 78.29) (end 192.725 77.775) (width 0.25) (layer "B.Cu") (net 8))
 (segment (start 156.76075 77.5) (end 153.5 80.76075) (width 0.5) (layer "B.Cu") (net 8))
 (segment (start 176.25 77.5) (end 156.76075 77.5) (width 0.5) (layer "B.Cu") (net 8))
 (segment (start 193.24 78.29) (end 205.74 78.29) (width 0.5) (layer "B.Cu") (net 8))
 (segment (start 190.45 75.5) (end 178.25 75.5) (width 0.5) (layer "B.Cu") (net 8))
 (segment (start 193.24 78.29) (end 193.2 78.25) (width 0.25) (layer "B.Cu") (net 8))
 (segment (start 208.2 81.75) (end 212.96 76.99) (width 0.5) (layer "B.Cu") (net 9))
 (segment (start 188.5 76.25) (end 194 81.75) (width 0.5) (layer "B.Cu") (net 9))
 (segment (start 212.96 89.49) (end 212.96 76.99) (width 0.5) (layer "B.Cu") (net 9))
 (segment (start 153.5 83.30075) (end 158.60075 78.2) (width 0.5) (layer "B.Cu") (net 9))
 (segment (start 194 81.75) (end 208.2 81.75) (width 0.5) (layer "B.Cu") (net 9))
 (segment (start 176.8 78.2) (end 178.75 76.25) (width 0.5) (layer "B.Cu") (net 9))
 (segment (start 158.60075 78.2) (end 176.8 78.2) (width 0.5) (layer "B.Cu") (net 9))
 (segment (start 178.75 76.25) (end 188.5 76.25) (width 0.5) (layer "B.Cu") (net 9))
 (segment (start 193.26 82.26) (end 188 77) (width 0.5) (layer "B.Cu") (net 10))
 (segment (start 177.35 78.9) (end 160.44075 78.9) (width 0.5) (layer "B.Cu") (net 10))
 (segment (start 193.26 88.21) (end 205.76 88.21) (width 0.5) (layer "B.Cu") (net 10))
 (segment (start 160.44075 78.9) (end 153.5 85.84075) (width 0.5) (layer "B.Cu") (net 10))
 (segment (start 188 77) (end 179.25 77) (width 0.5) (layer "B.Cu") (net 10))
 (segment (start 179.25 77) (end 177.35 78.9) (width 0.5) (layer "B.Cu") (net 10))
 (segment (start 193.26 88.21) (end 193.26 82.26) (width 0.5) (layer "B.Cu") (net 10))
 (segment (start 150.75 87) (end 152.13075 88.38075) (width 0.5) (layer "F.Cu") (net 11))
 (segment (start 150.75 85.25) (end 150.75 87) (width 0.5) (layer "F.Cu") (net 11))
 (segment (start 152.13075 88.38075) (end 153.5 88.38075) (width 0.5) (layer "F.Cu") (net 11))
 (segment (start 131.99 70.79) (end 144.49 70.79) (width 0.5) (layer "F.Cu") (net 11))
 (segment (start 144.49 78.99) (end 150.75 85.25) (width 0.5) (layer "F.Cu") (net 11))
 (segment (start 144.49 70.79) (end 144.49 78.99) (width 0.5) (layer "F.Cu") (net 11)))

